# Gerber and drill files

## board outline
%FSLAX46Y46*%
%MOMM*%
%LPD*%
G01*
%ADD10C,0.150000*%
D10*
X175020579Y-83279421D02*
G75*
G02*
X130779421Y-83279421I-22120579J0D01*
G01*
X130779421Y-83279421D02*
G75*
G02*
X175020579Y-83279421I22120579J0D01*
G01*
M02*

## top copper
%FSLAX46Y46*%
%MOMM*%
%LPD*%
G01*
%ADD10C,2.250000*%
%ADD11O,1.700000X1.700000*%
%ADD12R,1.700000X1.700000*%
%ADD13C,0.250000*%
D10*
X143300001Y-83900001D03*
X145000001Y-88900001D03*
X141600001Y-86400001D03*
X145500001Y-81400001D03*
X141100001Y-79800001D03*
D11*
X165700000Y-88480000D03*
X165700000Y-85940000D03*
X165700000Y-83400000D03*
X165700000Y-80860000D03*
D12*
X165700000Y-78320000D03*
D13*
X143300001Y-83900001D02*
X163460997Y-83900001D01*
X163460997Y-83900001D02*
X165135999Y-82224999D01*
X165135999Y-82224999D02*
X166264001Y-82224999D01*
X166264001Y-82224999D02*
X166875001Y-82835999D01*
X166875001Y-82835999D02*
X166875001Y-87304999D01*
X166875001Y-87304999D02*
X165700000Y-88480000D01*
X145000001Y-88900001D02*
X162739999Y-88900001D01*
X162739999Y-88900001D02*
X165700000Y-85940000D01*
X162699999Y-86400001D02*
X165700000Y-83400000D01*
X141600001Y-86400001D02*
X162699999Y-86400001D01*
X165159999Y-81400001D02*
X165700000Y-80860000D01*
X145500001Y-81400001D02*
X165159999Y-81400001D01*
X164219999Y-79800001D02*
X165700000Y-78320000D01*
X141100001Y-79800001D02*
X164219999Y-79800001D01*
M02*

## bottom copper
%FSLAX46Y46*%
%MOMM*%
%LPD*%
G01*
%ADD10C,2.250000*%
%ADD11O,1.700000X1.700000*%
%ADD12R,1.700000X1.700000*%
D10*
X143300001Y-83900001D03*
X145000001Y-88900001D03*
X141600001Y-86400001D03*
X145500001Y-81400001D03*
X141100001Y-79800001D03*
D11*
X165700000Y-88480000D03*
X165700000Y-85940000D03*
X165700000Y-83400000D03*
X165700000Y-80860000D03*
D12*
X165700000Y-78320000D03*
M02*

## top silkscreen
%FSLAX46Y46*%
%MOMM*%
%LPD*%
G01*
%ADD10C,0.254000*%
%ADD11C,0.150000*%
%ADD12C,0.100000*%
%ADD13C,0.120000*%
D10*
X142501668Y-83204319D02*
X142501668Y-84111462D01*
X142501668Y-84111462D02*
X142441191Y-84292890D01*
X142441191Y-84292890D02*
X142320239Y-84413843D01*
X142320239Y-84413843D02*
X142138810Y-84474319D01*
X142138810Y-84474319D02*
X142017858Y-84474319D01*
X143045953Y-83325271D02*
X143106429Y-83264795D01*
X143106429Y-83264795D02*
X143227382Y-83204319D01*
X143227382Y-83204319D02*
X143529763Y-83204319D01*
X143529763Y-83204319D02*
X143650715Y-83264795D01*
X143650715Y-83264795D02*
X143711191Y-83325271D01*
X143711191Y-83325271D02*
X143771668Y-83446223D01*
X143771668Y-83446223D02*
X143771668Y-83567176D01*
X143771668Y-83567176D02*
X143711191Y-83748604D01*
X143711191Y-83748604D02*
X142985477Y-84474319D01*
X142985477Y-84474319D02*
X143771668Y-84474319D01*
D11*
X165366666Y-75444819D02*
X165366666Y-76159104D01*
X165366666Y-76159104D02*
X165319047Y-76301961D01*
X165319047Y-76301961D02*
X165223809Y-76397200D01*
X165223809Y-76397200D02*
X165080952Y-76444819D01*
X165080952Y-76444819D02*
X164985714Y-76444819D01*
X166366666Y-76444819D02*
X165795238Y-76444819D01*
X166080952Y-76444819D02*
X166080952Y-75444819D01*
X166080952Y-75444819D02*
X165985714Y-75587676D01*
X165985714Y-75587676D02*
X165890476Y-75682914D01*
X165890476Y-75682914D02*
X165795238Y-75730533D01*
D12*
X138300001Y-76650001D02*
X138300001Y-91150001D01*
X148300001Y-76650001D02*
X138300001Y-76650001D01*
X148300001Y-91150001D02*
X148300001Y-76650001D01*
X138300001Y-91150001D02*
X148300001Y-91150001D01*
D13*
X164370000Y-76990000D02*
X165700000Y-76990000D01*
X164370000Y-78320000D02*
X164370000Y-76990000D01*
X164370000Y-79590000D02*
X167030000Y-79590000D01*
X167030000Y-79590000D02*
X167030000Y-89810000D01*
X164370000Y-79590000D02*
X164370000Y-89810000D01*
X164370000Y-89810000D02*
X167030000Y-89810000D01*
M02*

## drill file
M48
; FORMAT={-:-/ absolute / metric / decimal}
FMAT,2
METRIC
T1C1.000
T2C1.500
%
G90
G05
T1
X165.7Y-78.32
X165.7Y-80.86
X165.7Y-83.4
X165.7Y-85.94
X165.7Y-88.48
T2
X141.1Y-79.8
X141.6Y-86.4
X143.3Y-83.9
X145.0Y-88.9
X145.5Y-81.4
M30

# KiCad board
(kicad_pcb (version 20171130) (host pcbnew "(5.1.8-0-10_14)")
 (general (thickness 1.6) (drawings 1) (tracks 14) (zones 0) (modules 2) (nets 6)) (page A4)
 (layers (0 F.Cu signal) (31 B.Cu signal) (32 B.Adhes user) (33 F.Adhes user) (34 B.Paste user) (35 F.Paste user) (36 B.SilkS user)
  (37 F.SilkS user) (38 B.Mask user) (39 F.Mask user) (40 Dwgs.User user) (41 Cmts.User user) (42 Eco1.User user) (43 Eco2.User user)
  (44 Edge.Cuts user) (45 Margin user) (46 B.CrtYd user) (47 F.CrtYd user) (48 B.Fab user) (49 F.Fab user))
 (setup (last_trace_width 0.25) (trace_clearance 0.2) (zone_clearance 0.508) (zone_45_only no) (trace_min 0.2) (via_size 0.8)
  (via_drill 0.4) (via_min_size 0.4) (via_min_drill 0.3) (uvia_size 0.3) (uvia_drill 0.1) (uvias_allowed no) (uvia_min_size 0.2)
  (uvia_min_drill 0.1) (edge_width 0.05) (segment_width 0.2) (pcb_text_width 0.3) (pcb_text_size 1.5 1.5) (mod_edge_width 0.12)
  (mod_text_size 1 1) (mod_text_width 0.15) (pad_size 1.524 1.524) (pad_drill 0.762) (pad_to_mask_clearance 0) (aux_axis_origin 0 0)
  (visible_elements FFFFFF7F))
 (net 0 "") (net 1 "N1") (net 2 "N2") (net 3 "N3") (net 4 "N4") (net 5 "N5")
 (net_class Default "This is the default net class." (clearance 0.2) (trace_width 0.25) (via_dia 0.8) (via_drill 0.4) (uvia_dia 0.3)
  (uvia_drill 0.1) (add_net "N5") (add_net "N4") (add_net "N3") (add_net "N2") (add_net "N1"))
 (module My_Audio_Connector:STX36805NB (layer F.Cu) (at 141.100001 79.800001)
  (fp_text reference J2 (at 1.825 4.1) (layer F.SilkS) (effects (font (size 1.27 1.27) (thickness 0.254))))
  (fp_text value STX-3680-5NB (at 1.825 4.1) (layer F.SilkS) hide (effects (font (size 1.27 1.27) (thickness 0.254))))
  (fp_line (start -2.8 -3.15) (end -2.8 11.35) (layer F.SilkS) (width 0.1))
  (fp_line (start 7.2 -3.15) (end -2.8 -3.15) (layer F.SilkS) (width 0.1))
  (fp_line (start 7.2 11.35) (end 7.2 -3.15) (layer F.SilkS) (width 0.1))
  (fp_line (start -2.8 11.35) (end 7.2 11.35) (layer F.SilkS) (width 0.1))
  (pad S thru_hole circle (at 2.2 4.1) (size 2.25 2.25) (drill 1.5) (layers *.Cu *.Mask) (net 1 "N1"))
  (pad T thru_hole circle (at 3.9 9.1) (size 2.25 2.25) (drill 1.5) (layers *.Cu *.Mask) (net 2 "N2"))
  (pad TN thru_hole circle (at 0.5 6.6) (size 2.25 2.25) (drill 1.5) (layers *.Cu *.Mask) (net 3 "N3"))
  (pad RN thru_hole circle (at 4.4 1.6 90) (size 2.25 2.25) (drill 1.5) (layers *.Cu *.Mask) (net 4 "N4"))
  (pad R thru_hole circle (at 0 0) (size 2.25 2.25) (drill 1.5) (layers *.Cu *.Mask) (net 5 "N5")))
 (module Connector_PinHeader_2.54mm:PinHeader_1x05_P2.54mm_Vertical (layer F.Cu) (at 165.7 78.32)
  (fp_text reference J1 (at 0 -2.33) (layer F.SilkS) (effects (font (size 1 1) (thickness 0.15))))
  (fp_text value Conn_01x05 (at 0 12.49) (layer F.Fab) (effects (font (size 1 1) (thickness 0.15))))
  (fp_line (start -1.33 -1.33) (end 0 -1.33) (layer F.SilkS) (width 0.12))
  (fp_line (start -1.33 0) (end -1.33 -1.33) (layer F.SilkS) (width 0.12))
  (fp_line (start -1.33 1.27) (end 1.33 1.27) (layer F.SilkS) (width 0.12))
  (fp_line (start 1.33 1.27) (end 1.33 11.49) (layer F.SilkS) (width 0.12))
  (fp_line (start -1.33 1.27) (end -1.33 11.49) (layer F.SilkS) (width 0.12))
  (fp_line (start -1.33 11.49) (end 1.33 11.49) (layer F.SilkS) (width 0.12))
  (pad 5 thru_hole oval (at 0 10.16) (size 1.7 1.7) (drill 1) (layers *.Cu *.Mask) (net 1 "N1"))
  (pad 4 thru_hole oval (at 0 7.62) (size 1.7 1.7) (drill 1) (layers *.Cu *.Mask) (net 2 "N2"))
  (pad 3 thru_hole oval (at 0 5.08) (size 1.7 1.7) (drill 1) (layers *.Cu *.Mask) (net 3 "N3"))
  (pad 2 thru_hole oval (at 0 2.54) (size 1.7 1.7) (drill 1) (layers *.Cu *.Mask) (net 4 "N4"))
  (pad 1 thru_hole rect (at 0 0) (size 1.7 1.7) (drill 1) (layers *.Cu *.Mask) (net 5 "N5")))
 (gr_circle (center 152.9 83.279421) (end 175.020579 83.279421) (layer Edge.Cuts) (width 0.15))
 (segment (start 143.300001 83.900001) (end 163.460997 83.900001) (width 0.25) (layer F.Cu) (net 1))
 (segment (start 163.460997 83.900001) (end 165.135999 82.224999) (width 0.25) (layer F.Cu) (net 1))
 (segment (start 165.135999 82.224999) (end 166.264001 82.224999) (width 0.25) (layer F.Cu) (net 1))
 (segment (start 166.264001 82.224999) (end 166.875001 82.835999) (width 0.25) (layer F.Cu) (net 1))
 (segment (start 166.875001 82.835999) (end 166.875001 87.304999) (width 0.25) (layer F.Cu) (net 1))
 (segment (start 166.875001 87.304999) (end 165.7 88.48) (width 0.25) (layer F.Cu) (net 1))
 (segment (start 145.000001 88.900001) (end 162.739999 88.900001) (width 0.25) (layer F.Cu) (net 2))
 (segment (start 162.739999 88.900001) (end 165.7 85.94) (width 0.25) (layer F.Cu) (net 2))
 (segment (start 162.699999 86.400001) (end 165.7 83.4) (width 0.25) (layer F.Cu) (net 3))
 (segment (start 141.600001 86.400001) (end 162.699999 86.400001) (width 0.25) (layer F.Cu) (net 3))
 (segment (start 165.159999 81.400001) (end 165.7 80.86) (width 0.25) (layer F.Cu) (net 4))
 (segment (start 145.500001 81.400001) (end 165.159999 81.400001) (width 0.25) (layer F.Cu) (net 4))
 (segment (start 164.219999 79.800001) (end 165.7 78.32) (width 0.25) (layer F.Cu) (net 5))
 (segment (start 141.100001 79.800001) (end 164.219999 79.800001) (width 0.25) (layer F.Cu) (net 5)))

